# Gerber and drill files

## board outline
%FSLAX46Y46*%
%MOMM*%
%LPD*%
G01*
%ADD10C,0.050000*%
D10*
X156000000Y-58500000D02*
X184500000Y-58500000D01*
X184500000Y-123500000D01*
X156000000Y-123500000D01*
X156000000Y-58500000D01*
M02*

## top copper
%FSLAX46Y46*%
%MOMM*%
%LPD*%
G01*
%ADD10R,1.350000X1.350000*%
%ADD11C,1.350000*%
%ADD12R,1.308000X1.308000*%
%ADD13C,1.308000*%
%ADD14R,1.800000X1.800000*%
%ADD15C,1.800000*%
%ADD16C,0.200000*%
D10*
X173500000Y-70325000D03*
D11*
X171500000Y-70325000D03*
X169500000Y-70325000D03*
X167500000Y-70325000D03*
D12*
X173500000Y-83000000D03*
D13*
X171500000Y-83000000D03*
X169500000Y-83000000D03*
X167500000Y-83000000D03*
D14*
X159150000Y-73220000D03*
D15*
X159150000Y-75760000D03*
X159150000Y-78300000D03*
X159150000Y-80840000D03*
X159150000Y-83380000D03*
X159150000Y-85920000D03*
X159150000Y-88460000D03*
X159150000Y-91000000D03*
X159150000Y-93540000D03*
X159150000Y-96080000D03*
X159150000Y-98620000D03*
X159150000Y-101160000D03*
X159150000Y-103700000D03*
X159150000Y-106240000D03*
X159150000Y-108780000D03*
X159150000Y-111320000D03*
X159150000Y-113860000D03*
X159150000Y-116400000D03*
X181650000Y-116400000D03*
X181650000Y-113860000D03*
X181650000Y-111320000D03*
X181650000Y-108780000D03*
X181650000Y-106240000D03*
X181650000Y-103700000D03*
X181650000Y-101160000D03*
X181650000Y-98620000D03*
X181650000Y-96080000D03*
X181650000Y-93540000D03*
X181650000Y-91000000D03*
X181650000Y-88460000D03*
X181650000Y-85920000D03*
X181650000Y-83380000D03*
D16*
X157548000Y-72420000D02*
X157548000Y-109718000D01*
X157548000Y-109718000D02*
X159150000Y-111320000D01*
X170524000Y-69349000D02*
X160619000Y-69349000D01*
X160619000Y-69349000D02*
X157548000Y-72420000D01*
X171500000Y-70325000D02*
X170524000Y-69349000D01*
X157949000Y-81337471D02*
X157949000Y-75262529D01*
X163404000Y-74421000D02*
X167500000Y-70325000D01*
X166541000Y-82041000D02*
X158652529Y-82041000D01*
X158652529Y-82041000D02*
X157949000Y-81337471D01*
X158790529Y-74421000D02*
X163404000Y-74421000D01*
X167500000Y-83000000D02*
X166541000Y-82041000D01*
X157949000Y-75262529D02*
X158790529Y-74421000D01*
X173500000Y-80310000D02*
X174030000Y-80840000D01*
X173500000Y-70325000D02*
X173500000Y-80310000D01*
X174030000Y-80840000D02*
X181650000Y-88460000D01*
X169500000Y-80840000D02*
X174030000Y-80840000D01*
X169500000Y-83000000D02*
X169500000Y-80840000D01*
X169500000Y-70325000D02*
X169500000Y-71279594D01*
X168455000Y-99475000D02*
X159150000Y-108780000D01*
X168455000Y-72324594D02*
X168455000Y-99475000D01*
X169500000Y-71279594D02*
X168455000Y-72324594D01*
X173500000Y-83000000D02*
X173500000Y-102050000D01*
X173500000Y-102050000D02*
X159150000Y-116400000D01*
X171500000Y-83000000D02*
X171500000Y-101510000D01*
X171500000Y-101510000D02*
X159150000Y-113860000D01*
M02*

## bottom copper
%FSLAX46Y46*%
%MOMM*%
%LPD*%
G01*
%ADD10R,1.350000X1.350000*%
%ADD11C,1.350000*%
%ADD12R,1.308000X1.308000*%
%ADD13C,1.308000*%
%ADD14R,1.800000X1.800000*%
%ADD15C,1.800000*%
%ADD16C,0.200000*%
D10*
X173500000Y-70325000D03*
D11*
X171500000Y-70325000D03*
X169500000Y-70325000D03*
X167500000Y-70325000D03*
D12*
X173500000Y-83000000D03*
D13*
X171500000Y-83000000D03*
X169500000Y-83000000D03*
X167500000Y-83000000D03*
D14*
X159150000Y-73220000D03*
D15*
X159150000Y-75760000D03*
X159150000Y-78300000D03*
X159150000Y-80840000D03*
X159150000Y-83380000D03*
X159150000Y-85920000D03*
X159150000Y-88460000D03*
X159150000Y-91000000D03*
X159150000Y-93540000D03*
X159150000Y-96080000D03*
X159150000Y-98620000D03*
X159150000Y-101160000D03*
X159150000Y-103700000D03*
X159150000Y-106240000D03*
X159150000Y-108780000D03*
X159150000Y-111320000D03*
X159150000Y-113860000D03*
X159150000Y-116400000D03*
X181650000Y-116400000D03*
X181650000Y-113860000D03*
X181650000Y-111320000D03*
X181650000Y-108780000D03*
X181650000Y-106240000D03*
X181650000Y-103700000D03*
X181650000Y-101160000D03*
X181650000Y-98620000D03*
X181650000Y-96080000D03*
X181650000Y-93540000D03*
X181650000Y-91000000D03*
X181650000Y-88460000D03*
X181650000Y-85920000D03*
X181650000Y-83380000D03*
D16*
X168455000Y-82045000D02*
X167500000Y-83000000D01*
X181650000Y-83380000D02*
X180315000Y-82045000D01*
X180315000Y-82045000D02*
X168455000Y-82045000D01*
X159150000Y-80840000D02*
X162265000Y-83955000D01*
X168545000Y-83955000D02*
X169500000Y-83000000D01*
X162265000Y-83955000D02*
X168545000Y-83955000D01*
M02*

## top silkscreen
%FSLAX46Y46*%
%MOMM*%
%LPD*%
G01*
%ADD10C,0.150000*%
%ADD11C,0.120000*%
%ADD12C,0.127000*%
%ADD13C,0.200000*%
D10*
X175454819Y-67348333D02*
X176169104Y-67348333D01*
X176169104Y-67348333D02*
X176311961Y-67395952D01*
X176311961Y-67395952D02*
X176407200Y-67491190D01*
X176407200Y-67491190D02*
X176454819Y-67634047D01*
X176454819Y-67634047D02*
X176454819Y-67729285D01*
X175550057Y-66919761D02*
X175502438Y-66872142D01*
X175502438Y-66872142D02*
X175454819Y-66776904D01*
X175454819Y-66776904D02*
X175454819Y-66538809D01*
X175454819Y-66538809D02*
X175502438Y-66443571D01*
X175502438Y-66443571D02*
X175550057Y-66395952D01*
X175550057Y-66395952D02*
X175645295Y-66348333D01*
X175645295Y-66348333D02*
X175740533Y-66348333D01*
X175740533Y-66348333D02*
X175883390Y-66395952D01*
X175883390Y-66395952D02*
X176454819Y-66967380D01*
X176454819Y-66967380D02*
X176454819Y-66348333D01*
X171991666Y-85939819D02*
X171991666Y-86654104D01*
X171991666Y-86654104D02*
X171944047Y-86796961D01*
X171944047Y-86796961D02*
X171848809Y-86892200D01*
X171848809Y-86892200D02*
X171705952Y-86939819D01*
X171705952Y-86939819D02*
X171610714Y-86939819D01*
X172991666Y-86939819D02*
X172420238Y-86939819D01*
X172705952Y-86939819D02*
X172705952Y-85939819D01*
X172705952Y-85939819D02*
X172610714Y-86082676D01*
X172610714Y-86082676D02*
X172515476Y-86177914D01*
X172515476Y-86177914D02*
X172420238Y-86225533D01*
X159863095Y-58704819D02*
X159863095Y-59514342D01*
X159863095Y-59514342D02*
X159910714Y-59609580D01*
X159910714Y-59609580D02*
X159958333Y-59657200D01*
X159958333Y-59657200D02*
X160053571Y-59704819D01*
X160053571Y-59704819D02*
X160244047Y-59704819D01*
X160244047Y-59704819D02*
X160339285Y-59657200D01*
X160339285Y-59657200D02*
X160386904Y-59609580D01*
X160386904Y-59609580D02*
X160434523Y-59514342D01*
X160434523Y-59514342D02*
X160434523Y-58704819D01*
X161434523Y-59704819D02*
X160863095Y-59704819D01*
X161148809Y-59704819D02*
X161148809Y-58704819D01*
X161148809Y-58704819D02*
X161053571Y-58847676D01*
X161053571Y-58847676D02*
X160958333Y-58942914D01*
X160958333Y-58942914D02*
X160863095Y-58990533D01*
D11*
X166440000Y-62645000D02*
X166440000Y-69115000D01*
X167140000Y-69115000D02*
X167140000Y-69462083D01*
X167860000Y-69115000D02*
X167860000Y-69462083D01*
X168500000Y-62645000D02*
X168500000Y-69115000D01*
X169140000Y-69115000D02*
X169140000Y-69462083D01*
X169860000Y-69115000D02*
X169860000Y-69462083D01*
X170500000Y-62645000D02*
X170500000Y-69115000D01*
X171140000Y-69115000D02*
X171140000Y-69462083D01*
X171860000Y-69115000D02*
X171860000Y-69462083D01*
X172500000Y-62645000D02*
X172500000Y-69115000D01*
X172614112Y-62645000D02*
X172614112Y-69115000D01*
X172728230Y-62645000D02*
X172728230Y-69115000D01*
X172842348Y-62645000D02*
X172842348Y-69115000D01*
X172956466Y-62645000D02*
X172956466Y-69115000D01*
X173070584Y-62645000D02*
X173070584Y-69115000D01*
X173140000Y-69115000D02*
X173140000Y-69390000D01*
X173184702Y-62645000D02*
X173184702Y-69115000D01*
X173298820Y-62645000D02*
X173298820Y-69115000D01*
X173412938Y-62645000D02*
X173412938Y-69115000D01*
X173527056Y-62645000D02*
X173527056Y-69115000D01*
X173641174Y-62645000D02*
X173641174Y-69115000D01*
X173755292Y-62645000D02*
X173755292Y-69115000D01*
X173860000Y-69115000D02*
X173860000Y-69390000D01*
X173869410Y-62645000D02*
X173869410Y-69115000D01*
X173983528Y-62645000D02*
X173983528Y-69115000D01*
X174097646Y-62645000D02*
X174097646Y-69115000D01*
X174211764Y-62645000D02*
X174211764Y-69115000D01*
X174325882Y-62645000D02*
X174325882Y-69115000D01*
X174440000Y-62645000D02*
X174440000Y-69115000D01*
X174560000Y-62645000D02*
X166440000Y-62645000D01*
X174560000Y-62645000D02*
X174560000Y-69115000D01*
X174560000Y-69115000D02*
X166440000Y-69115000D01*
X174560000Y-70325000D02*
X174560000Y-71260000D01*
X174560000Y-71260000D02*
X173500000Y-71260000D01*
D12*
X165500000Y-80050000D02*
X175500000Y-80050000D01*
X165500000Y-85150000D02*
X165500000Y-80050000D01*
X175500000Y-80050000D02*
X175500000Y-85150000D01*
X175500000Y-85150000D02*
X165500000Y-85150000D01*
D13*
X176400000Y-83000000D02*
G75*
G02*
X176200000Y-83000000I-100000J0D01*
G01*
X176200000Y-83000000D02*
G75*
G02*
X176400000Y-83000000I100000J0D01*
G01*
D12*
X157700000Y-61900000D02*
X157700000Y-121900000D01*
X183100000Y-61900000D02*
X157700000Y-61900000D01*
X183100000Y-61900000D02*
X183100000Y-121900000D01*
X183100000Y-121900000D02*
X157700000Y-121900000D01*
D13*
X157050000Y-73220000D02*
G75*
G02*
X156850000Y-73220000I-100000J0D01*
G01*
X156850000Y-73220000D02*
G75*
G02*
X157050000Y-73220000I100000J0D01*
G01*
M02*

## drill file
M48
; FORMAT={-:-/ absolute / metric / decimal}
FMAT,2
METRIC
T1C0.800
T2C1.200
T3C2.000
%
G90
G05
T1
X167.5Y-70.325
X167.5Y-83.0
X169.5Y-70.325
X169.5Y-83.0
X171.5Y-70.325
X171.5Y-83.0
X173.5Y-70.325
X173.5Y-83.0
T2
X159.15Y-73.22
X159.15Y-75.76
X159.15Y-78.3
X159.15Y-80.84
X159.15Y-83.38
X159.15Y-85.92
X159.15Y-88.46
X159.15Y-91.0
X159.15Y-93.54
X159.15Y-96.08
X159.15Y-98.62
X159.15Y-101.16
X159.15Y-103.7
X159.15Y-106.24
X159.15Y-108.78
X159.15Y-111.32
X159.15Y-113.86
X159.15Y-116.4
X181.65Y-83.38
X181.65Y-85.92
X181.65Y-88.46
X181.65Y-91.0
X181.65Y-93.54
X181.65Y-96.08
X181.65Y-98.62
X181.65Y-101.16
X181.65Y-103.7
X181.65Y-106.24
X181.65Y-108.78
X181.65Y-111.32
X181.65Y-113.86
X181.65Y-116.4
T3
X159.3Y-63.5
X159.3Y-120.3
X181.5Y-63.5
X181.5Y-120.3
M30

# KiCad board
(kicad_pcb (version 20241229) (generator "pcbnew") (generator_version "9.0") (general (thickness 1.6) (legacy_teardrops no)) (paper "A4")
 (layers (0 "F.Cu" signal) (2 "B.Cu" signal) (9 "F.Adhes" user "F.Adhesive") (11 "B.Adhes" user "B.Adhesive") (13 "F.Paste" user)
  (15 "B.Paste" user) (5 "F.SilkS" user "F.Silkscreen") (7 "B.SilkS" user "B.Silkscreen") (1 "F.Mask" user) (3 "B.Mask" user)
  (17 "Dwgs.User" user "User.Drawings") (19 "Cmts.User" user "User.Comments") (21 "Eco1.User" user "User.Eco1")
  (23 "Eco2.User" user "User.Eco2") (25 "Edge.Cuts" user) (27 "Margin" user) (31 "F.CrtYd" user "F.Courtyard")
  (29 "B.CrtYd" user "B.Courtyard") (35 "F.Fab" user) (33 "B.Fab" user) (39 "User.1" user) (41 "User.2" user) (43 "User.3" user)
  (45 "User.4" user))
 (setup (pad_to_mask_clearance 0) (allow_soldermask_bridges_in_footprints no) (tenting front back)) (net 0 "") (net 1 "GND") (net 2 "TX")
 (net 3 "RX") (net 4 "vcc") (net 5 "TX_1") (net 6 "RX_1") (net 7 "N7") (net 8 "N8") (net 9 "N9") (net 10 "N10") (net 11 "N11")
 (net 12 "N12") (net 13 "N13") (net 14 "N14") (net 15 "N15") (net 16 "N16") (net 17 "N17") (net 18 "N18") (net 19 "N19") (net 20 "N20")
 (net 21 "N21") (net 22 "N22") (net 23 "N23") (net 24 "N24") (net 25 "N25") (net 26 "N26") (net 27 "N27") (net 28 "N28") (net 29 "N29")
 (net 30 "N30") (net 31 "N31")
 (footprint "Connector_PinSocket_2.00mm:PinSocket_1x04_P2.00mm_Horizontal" (layer "F.Cu") (at 173.5 70.325 -90)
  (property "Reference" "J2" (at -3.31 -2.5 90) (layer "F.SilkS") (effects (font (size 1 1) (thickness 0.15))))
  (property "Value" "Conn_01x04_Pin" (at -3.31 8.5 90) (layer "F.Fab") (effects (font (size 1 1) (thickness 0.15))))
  (fp_line (start -7.68 7.06) (end -1.21 7.06) (stroke (width 0.12) (type solid)) (layer "F.SilkS"))
  (fp_line (start -1.21 6.36) (end -0.862917 6.36) (stroke (width 0.12) (type solid)) (layer "F.SilkS"))
  (fp_line (start -1.21 5.64) (end -0.862917 5.64) (stroke (width 0.12) (type solid)) (layer "F.SilkS"))
  (fp_line (start -7.68 5) (end -1.21 5) (stroke (width 0.12) (type solid)) (layer "F.SilkS"))
  (fp_line (start -1.21 4.36) (end -0.862917 4.36) (stroke (width 0.12) (type solid)) (layer "F.SilkS"))
  (fp_line (start -1.21 3.64) (end -0.862917 3.64) (stroke (width 0.12) (type solid)) (layer "F.SilkS"))
  (fp_line (start -7.68 3) (end -1.21 3) (stroke (width 0.12) (type solid)) (layer "F.SilkS"))
  (fp_line (start -1.21 2.36) (end -0.862917 2.36) (stroke (width 0.12) (type solid)) (layer "F.SilkS"))
  (fp_line (start -1.21 1.64) (end -0.862917 1.64) (stroke (width 0.12) (type solid)) (layer "F.SilkS"))
  (fp_line (start -7.68 1) (end -1.21 1) (stroke (width 0.12) (type solid)) (layer "F.SilkS"))
  (fp_line (start -7.68 0.885888) (end -1.21 0.885888) (stroke (width 0.12) (type solid)) (layer "F.SilkS"))
  (fp_line (start -7.68 0.77177) (end -1.21 0.77177) (stroke (width 0.12) (type solid)) (layer "F.SilkS"))
  (fp_line (start -7.68 0.657652) (end -1.21 0.657652) (stroke (width 0.12) (type solid)) (layer "F.SilkS"))
  (fp_line (start -7.68 0.543534) (end -1.21 0.543534) (stroke (width 0.12) (type solid)) (layer "F.SilkS"))
  (fp_line (start -7.68 0.429416) (end -1.21 0.429416) (stroke (width 0.12) (type solid)) (layer "F.SilkS"))
  (fp_line (start -1.21 0.36) (end -0.935 0.36) (stroke (width 0.12) (type solid)) (layer "F.SilkS"))
  (fp_line (start -7.68 0.315298) (end -1.21 0.315298) (stroke (width 0.12) (type solid)) (layer "F.SilkS"))
  (fp_line (start -7.68 0.20118) (end -1.21 0.20118) (stroke (width 0.12) (type solid)) (layer "F.SilkS"))
  (fp_line (start -7.68 0.087062) (end -1.21 0.087062) (stroke (width 0.12) (type solid)) (layer "F.SilkS"))
  (fp_line (start -7.68 -0.027056) (end -1.21 -0.027056) (stroke (width 0.12) (type solid)) (layer "F.SilkS"))
  (fp_line (start -7.68 -0.141174) (end -1.21 -0.141174) (stroke (width 0.12) (type solid)) (layer "F.SilkS"))
  (fp_line (start -7.68 -0.255292) (end -1.21 -0.255292) (stroke (width 0.12) (type solid)) (layer "F.SilkS"))
  (fp_line (start -1.21 -0.36) (end -0.935 -0.36) (stroke (width 0.12) (type solid)) (layer "F.SilkS"))
  (fp_line (start -7.68 -0.36941) (end -1.21 -0.36941) (stroke (width 0.12) (type solid)) (layer "F.SilkS"))
  (fp_line (start -7.68 -0.483528) (end -1.21 -0.483528) (stroke (width 0.12) (type solid)) (layer "F.SilkS"))
  (fp_line (start -7.68 -0.597646) (end -1.21 -0.597646) (stroke (width 0.12) (type solid)) (layer "F.SilkS"))
  (fp_line (start -7.68 -0.711764) (end -1.21 -0.711764) (stroke (width 0.12) (type solid)) (layer "F.SilkS"))
  (fp_line (start -7.68 -0.825882) (end -1.21 -0.825882) (stroke (width 0.12) (type solid)) (layer "F.SilkS"))
  (fp_line (start -7.68 -0.94) (end -1.21 -0.94) (stroke (width 0.12) (type solid)) (layer "F.SilkS"))
  (fp_line (start -7.68 -1.06) (end -7.68 7.06) (stroke (width 0.12) (type solid)) (layer "F.SilkS"))
  (fp_line (start -7.68 -1.06) (end -1.21 -1.06) (stroke (width 0.12) (type solid)) (layer "F.SilkS"))
  (fp_line (start -1.21 -1.06) (end -1.21 7.06) (stroke (width 0.12) (type solid)) (layer "F.SilkS"))
  (fp_line (start 0 -1.06) (end 0.935 -1.06) (stroke (width 0.12) (type solid)) (layer "F.SilkS"))
  (fp_line (start 0.935 -1.06) (end 0.935 0) (stroke (width 0.12) (type solid)) (layer "F.SilkS"))
  (pad "1" thru_hole rect (at 0 0 270) (size 1.35 1.35) (drill 0.8) (layers "*.Cu" "*.Mask") (remove_unused_layers no) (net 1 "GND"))
  (pad "2" thru_hole circle (at 0 2 270) (size 1.35 1.35) (drill 0.8) (layers "*.Cu" "*.Mask") (remove_unused_layers no) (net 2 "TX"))
  (pad "3" thru_hole circle (at 0 4 270) (size 1.35 1.35) (drill 0.8) (layers "*.Cu" "*.Mask") (remove_unused_layers no) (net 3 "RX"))
  (pad "4" thru_hole circle (at 0 6 270) (size 1.35 1.35) (drill 0.8) (layers "*.Cu" "*.Mask") (remove_unused_layers no) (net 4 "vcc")))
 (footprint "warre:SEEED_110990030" (layer "F.Cu") (at 170.5 83 180)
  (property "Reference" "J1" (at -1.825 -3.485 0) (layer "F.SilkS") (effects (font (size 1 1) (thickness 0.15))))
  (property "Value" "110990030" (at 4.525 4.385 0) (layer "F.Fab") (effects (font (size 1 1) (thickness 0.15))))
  (fp_line (start 5 2.95) (end -5 2.95) (stroke (width 0.127) (type solid)) (layer "F.SilkS"))
  (fp_line (start 5 -2.15) (end 5 2.95) (stroke (width 0.127) (type solid)) (layer "F.SilkS"))
  (fp_line (start -5 2.95) (end -5 -2.15) (stroke (width 0.127) (type solid)) (layer "F.SilkS"))
  (fp_line (start -5 -2.15) (end 5 -2.15) (stroke (width 0.127) (type solid)) (layer "F.SilkS"))
  (fp_circle (center -5.8 0) (end -5.7 0) (stroke (width 0.2) (type solid)) (fill no) (layer "F.SilkS"))
  (pad "1" thru_hole rect (at -3 0 180) (size 1.308 1.308) (drill 0.8) (layers "*.Cu" "*.Mask") (remove_unused_layers no) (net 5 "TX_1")
   (solder_mask_margin 0.102))
  (pad "2" thru_hole circle (at -1 0 180) (size 1.308 1.308) (drill 0.8) (layers "*.Cu" "*.Mask") (remove_unused_layers no) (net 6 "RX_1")
   (solder_mask_margin 0.102))
  (pad "3" thru_hole circle (at 1 0 180) (size 1.308 1.308) (drill 0.8) (layers "*.Cu" "*.Mask") (remove_unused_layers no) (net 1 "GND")
   (solder_mask_margin 0.102))
  (pad "4" thru_hole circle (at 3 0 180) (size 1.308 1.308) (drill 0.8) (layers "*.Cu" "*.Mask") (remove_unused_layers no) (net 4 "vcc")
   (solder_mask_margin 0.102)))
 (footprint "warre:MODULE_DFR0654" (layer "F.Cu") (at 170.4 91.9)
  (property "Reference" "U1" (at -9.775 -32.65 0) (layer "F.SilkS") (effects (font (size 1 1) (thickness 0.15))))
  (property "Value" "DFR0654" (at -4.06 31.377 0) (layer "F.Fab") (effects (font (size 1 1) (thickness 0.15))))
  (fp_line (start -12.7 -30) (end -12.7 30) (stroke (width 0.127) (type solid)) (layer "F.SilkS"))
  (fp_line (start 12.7 -30) (end -12.7 -30) (stroke (width 0.127) (type solid)) (layer "F.SilkS"))
  (fp_line (start 12.7 -30) (end 12.7 30) (stroke (width 0.127) (type solid)) (layer "F.SilkS"))
  (fp_line (start 12.7 30) (end -12.7 30) (stroke (width 0.127) (type solid)) (layer "F.SilkS"))
  (fp_circle (center -13.45 -18.68) (end -13.35 -18.68) (stroke (width 0.2) (type solid)) (fill no) (layer "F.SilkS"))
  (pad "" np_thru_hole circle (at -11.1 -28.4) (size 2 2) (drill 2) (layers "*.Cu" "*.Mask"))
  (pad "" np_thru_hole circle (at -11.1 28.4) (size 2 2) (drill 2) (layers "*.Cu" "*.Mask"))
  (pad "" np_thru_hole circle (at 11.1 -28.4) (size 2 2) (drill 2) (layers "*.Cu" "*.Mask"))
  (pad "" np_thru_hole circle (at 11.1 28.4) (size 2 2) (drill 2) (layers "*.Cu" "*.Mask"))
  (pad "1" thru_hole rect (at -11.25 -18.68) (size 1.8 1.8) (drill 1.2) (layers "*.Cu" "*.Mask") (remove_unused_layers no) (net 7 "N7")
   (solder_mask_margin 0.102))
  (pad "2" thru_hole circle (at -11.25 -16.14) (size 1.8 1.8) (drill 1.2) (layers "*.Cu" "*.Mask") (remove_unused_layers no) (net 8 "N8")
   (solder_mask_margin 0.102))
  (pad "3" thru_hole circle (at -11.25 -13.6) (size 1.8 1.8) (drill 1.2) (layers "*.Cu" "*.Mask") (remove_unused_layers no) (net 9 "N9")
   (solder_mask_margin 0.102))
  (pad "4" thru_hole circle (at -11.25 -11.06) (size 1.8 1.8) (drill 1.2) (layers "*.Cu" "*.Mask") (remove_unused_layers no) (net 1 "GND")
   (solder_mask_margin 0.102))
  (pad "5" thru_hole circle (at -11.25 -8.52) (size 1.8 1.8) (drill 1.2) (layers "*.Cu" "*.Mask") (remove_unused_layers no) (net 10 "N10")
   (solder_mask_margin 0.102))
  (pad "6" thru_hole circle (at -11.25 -5.98) (size 1.8 1.8) (drill 1.2) (layers "*.Cu" "*.Mask") (remove_unused_layers no) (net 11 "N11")
   (solder_mask_margin 0.102))
  (pad "7" thru_hole circle (at -11.25 -3.44) (size 1.8 1.8) (drill 1.2) (layers "*.Cu" "*.Mask") (remove_unused_layers no) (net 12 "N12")
   (solder_mask_margin 0.102))
  (pad "8" thru_hole circle (at -11.25 -0.9) (size 1.8 1.8) (drill 1.2) (layers "*.Cu" "*.Mask") (remove_unused_layers no) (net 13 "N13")
   (solder_mask_margin 0.102))
  (pad "9" thru_hole circle (at -11.25 1.64) (size 1.8 1.8) (drill 1.2) (layers "*.Cu" "*.Mask") (remove_unused_layers no) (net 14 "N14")
   (solder_mask_margin 0.102))
  (pad "10" thru_hole circle (at -11.25 4.18) (size 1.8 1.8) (drill 1.2) (layers "*.Cu" "*.Mask") (remove_unused_layers no) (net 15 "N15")
   (solder_mask_margin 0.102))
  (pad "11" thru_hole circle (at -11.25 6.72) (size 1.8 1.8) (drill 1.2) (layers "*.Cu" "*.Mask") (remove_unused_layers no) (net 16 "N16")
   (solder_mask_margin 0.102))
  (pad "12" thru_hole circle (at -11.25 9.26) (size 1.8 1.8) (drill 1.2) (layers "*.Cu" "*.Mask") (remove_unused_layers no) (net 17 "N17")
   (solder_mask_margin 0.102))
  (pad "13" thru_hole circle (at -11.25 11.8) (size 1.8 1.8) (drill 1.2) (layers "*.Cu" "*.Mask") (remove_unused_layers no) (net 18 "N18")
   (solder_mask_margin 0.102))
  (pad "14" thru_hole circle (at -11.25 14.34) (size 1.8 1.8) (drill 1.2) (layers "*.Cu" "*.Mask") (remove_unused_layers no) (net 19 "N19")
   (solder_mask_margin 0.102))
  (pad "15" thru_hole circle (at -11.25 16.88) (size 1.8 1.8) (drill 1.2) (layers "*.Cu" "*.Mask") (remove_unused_layers no) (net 3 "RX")
   (solder_mask_margin 0.102))
  (pad "16" thru_hole circle (at -11.25 19.42) (size 1.8 1.8) (drill 1.2) (layers "*.Cu" "*.Mask") (remove_unused_layers no) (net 2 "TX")
   (solder_mask_margin 0.102))
  (pad "17" thru_hole circle (at -11.25 21.96) (size 1.8 1.8) (drill 1.2) (layers "*.Cu" "*.Mask") (remove_unused_layers no) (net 6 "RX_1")
   (solder_mask_margin 0.102))
  (pad "18" thru_hole circle (at -11.25 24.5) (size 1.8 1.8) (drill 1.2) (layers "*.Cu" "*.Mask") (remove_unused_layers no) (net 5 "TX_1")
   (solder_mask_margin 0.102))
  (pad "19" thru_hole circle (at 11.25 24.5) (size 1.8 1.8) (drill 1.2) (layers "*.Cu" "*.Mask") (remove_unused_layers no) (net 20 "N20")
   (solder_mask_margin 0.102))
  (pad "20" thru_hole circle (at 11.25 21.96) (size 1.8 1.8) (drill 1.2) (layers "*.Cu" "*.Mask") (remove_unused_layers no) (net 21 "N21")
   (solder_mask_margin 0.102))
  (pad "21" thru_hole circle (at 11.25 19.42) (size 1.8 1.8) (drill 1.2) (layers "*.Cu" "*.Mask") (remove_unused_layers no) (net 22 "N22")
   (solder_mask_margin 0.102))
  (pad "22" thru_hole circle (at 11.25 16.88) (size 1.8 1.8) (drill 1.2) (layers "*.Cu" "*.Mask") (remove_unused_layers no) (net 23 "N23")
   (solder_mask_margin 0.102))
  (pad "23" thru_hole circle (at 11.25 14.34) (size 1.8 1.8) (drill 1.2) (layers "*.Cu" "*.Mask") (remove_unused_layers no) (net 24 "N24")
   (solder_mask_margin 0.102))
  (pad "24" thru_hole circle (at 11.25 11.8) (size 1.8 1.8) (drill 1.2) (layers "*.Cu" "*.Mask") (remove_unused_layers no) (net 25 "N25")
   (solder_mask_margin 0.102))
  (pad "25" thru_hole circle (at 11.25 9.26) (size 1.8 1.8) (drill 1.2) (layers "*.Cu" "*.Mask") (remove_unused_layers no) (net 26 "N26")
   (solder_mask_margin 0.102))
  (pad "26" thru_hole circle (at 11.25 6.72) (size 1.8 1.8) (drill 1.2) (layers "*.Cu" "*.Mask") (remove_unused_layers no) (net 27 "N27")
   (solder_mask_margin 0.102))
  (pad "27" thru_hole circle (at 11.25 4.18) (size 1.8 1.8) (drill 1.2) (layers "*.Cu" "*.Mask") (remove_unused_layers no) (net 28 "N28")
   (solder_mask_margin 0.102))
  (pad "28" thru_hole circle (at 11.25 1.64) (size 1.8 1.8) (drill 1.2) (layers "*.Cu" "*.Mask") (remove_unused_layers no) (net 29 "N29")
   (solder_mask_margin 0.102))
  (pad "29" thru_hole circle (at 11.25 -0.9) (size 1.8 1.8) (drill 1.2) (layers "*.Cu" "*.Mask") (remove_unused_layers no) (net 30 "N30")
   (solder_mask_margin 0.102))
  (pad "30" thru_hole circle (at 11.25 -3.44) (size 1.8 1.8) (drill 1.2) (layers "*.Cu" "*.Mask") (remove_unused_layers no) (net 1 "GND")
   (solder_mask_margin 0.102))
  (pad "31" thru_hole circle (at 11.25 -5.98) (size 1.8 1.8) (drill 1.2) (layers "*.Cu" "*.Mask") (remove_unused_layers no) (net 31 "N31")
   (solder_mask_margin 0.102))
  (pad "32" thru_hole circle (at 11.25 -8.52) (size 1.8 1.8) (drill 1.2) (layers "*.Cu" "*.Mask") (remove_unused_layers no) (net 4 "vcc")
   (solder_mask_margin 0.102)))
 (gr_rect (start 156 58.5) (end 184.5 123.5) (stroke (width 0.05) (type default)) (fill no) (layer "Edge.Cuts"))
 (segment (start 157.548 72.42) (end 157.548 109.718) (width 0.2) (layer "F.Cu") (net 2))
 (segment (start 157.548 109.718) (end 159.15 111.32) (width 0.2) (layer "F.Cu") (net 2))
 (segment (start 170.524 69.349) (end 160.619 69.349) (width 0.2) (layer "F.Cu") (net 2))
 (segment (start 160.619 69.349) (end 157.548 72.42) (width 0.2) (layer "F.Cu") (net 2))
 (segment (start 171.5 70.325) (end 170.524 69.349) (width 0.2) (layer "F.Cu") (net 2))
 (segment (start 157.949 81.337471) (end 157.949 75.262529) (width 0.2) (layer "F.Cu") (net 4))
 (segment (start 163.404 74.421) (end 167.5 70.325) (width 0.2) (layer "F.Cu") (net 4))
 (segment (start 166.541 82.041) (end 158.652529 82.041) (width 0.2) (layer "F.Cu") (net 4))
 (segment (start 158.652529 82.041) (end 157.949 81.337471) (width 0.2) (layer "F.Cu") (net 4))
 (segment (start 158.790529 74.421) (end 163.404 74.421) (width 0.2) (layer "F.Cu") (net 4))
 (segment (start 167.5 83) (end 166.541 82.041) (width 0.2) (layer "F.Cu") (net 4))
 (segment (start 157.949 75.262529) (end 158.790529 74.421) (width 0.2) (layer "F.Cu") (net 4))
 (segment (start 168.455 82.045) (end 167.5 83) (width 0.2) (layer "B.Cu") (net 4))
 (segment (start 181.65 83.38) (end 180.315 82.045) (width 0.2) (layer "B.Cu") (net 4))
 (segment (start 180.315 82.045) (end 168.455 82.045) (width 0.2) (layer "B.Cu") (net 4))
 (segment (start 173.5 80.31) (end 174.03 80.84) (width 0.2) (layer "F.Cu") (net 1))
 (segment (start 173.5 70.325) (end 173.5 80.31) (width 0.2) (layer "F.Cu") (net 1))
 (segment (start 174.03 80.84) (end 181.65 88.46) (width 0.2) (layer "F.Cu") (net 1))
 (segment (start 169.5 80.84) (end 174.03 80.84) (width 0.2) (layer "F.Cu") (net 1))
 (segment (start 169.5 83) (end 169.5 80.84) (width 0.2) (layer "F.Cu") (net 1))
 (segment (start 159.15 80.84) (end 162.265 83.955) (width 0.2) (layer "B.Cu") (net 1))
 (segment (start 168.545 83.955) (end 169.5 83) (width 0.2) (layer "B.Cu") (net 1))
 (segment (start 162.265 83.955) (end 168.545 83.955) (width 0.2) (layer "B.Cu") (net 1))
 (segment (start 169.5 70.325) (end 169.5 71.279594) (width 0.2) (layer "F.Cu") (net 3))
 (segment (start 168.455 99.475) (end 159.15 108.78) (width 0.2) (layer "F.Cu") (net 3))
 (segment (start 168.455 72.324594) (end 168.455 99.475) (width 0.2) (layer "F.Cu") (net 3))
 (segment (start 169.5 71.279594) (end 168.455 72.324594) (width 0.2) (layer "F.Cu") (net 3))
 (segment (start 173.5 83) (end 173.5 102.05) (width 0.2) (layer "F.Cu") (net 5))
 (segment (start 173.5 102.05) (end 159.15 116.4) (width 0.2) (layer "F.Cu") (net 5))
 (segment (start 171.5 83) (end 171.5 101.51) (width 0.2) (layer "F.Cu") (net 6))
 (segment (start 171.5 101.51) (end 159.15 113.86) (width 0.2) (layer "F.Cu") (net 6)))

